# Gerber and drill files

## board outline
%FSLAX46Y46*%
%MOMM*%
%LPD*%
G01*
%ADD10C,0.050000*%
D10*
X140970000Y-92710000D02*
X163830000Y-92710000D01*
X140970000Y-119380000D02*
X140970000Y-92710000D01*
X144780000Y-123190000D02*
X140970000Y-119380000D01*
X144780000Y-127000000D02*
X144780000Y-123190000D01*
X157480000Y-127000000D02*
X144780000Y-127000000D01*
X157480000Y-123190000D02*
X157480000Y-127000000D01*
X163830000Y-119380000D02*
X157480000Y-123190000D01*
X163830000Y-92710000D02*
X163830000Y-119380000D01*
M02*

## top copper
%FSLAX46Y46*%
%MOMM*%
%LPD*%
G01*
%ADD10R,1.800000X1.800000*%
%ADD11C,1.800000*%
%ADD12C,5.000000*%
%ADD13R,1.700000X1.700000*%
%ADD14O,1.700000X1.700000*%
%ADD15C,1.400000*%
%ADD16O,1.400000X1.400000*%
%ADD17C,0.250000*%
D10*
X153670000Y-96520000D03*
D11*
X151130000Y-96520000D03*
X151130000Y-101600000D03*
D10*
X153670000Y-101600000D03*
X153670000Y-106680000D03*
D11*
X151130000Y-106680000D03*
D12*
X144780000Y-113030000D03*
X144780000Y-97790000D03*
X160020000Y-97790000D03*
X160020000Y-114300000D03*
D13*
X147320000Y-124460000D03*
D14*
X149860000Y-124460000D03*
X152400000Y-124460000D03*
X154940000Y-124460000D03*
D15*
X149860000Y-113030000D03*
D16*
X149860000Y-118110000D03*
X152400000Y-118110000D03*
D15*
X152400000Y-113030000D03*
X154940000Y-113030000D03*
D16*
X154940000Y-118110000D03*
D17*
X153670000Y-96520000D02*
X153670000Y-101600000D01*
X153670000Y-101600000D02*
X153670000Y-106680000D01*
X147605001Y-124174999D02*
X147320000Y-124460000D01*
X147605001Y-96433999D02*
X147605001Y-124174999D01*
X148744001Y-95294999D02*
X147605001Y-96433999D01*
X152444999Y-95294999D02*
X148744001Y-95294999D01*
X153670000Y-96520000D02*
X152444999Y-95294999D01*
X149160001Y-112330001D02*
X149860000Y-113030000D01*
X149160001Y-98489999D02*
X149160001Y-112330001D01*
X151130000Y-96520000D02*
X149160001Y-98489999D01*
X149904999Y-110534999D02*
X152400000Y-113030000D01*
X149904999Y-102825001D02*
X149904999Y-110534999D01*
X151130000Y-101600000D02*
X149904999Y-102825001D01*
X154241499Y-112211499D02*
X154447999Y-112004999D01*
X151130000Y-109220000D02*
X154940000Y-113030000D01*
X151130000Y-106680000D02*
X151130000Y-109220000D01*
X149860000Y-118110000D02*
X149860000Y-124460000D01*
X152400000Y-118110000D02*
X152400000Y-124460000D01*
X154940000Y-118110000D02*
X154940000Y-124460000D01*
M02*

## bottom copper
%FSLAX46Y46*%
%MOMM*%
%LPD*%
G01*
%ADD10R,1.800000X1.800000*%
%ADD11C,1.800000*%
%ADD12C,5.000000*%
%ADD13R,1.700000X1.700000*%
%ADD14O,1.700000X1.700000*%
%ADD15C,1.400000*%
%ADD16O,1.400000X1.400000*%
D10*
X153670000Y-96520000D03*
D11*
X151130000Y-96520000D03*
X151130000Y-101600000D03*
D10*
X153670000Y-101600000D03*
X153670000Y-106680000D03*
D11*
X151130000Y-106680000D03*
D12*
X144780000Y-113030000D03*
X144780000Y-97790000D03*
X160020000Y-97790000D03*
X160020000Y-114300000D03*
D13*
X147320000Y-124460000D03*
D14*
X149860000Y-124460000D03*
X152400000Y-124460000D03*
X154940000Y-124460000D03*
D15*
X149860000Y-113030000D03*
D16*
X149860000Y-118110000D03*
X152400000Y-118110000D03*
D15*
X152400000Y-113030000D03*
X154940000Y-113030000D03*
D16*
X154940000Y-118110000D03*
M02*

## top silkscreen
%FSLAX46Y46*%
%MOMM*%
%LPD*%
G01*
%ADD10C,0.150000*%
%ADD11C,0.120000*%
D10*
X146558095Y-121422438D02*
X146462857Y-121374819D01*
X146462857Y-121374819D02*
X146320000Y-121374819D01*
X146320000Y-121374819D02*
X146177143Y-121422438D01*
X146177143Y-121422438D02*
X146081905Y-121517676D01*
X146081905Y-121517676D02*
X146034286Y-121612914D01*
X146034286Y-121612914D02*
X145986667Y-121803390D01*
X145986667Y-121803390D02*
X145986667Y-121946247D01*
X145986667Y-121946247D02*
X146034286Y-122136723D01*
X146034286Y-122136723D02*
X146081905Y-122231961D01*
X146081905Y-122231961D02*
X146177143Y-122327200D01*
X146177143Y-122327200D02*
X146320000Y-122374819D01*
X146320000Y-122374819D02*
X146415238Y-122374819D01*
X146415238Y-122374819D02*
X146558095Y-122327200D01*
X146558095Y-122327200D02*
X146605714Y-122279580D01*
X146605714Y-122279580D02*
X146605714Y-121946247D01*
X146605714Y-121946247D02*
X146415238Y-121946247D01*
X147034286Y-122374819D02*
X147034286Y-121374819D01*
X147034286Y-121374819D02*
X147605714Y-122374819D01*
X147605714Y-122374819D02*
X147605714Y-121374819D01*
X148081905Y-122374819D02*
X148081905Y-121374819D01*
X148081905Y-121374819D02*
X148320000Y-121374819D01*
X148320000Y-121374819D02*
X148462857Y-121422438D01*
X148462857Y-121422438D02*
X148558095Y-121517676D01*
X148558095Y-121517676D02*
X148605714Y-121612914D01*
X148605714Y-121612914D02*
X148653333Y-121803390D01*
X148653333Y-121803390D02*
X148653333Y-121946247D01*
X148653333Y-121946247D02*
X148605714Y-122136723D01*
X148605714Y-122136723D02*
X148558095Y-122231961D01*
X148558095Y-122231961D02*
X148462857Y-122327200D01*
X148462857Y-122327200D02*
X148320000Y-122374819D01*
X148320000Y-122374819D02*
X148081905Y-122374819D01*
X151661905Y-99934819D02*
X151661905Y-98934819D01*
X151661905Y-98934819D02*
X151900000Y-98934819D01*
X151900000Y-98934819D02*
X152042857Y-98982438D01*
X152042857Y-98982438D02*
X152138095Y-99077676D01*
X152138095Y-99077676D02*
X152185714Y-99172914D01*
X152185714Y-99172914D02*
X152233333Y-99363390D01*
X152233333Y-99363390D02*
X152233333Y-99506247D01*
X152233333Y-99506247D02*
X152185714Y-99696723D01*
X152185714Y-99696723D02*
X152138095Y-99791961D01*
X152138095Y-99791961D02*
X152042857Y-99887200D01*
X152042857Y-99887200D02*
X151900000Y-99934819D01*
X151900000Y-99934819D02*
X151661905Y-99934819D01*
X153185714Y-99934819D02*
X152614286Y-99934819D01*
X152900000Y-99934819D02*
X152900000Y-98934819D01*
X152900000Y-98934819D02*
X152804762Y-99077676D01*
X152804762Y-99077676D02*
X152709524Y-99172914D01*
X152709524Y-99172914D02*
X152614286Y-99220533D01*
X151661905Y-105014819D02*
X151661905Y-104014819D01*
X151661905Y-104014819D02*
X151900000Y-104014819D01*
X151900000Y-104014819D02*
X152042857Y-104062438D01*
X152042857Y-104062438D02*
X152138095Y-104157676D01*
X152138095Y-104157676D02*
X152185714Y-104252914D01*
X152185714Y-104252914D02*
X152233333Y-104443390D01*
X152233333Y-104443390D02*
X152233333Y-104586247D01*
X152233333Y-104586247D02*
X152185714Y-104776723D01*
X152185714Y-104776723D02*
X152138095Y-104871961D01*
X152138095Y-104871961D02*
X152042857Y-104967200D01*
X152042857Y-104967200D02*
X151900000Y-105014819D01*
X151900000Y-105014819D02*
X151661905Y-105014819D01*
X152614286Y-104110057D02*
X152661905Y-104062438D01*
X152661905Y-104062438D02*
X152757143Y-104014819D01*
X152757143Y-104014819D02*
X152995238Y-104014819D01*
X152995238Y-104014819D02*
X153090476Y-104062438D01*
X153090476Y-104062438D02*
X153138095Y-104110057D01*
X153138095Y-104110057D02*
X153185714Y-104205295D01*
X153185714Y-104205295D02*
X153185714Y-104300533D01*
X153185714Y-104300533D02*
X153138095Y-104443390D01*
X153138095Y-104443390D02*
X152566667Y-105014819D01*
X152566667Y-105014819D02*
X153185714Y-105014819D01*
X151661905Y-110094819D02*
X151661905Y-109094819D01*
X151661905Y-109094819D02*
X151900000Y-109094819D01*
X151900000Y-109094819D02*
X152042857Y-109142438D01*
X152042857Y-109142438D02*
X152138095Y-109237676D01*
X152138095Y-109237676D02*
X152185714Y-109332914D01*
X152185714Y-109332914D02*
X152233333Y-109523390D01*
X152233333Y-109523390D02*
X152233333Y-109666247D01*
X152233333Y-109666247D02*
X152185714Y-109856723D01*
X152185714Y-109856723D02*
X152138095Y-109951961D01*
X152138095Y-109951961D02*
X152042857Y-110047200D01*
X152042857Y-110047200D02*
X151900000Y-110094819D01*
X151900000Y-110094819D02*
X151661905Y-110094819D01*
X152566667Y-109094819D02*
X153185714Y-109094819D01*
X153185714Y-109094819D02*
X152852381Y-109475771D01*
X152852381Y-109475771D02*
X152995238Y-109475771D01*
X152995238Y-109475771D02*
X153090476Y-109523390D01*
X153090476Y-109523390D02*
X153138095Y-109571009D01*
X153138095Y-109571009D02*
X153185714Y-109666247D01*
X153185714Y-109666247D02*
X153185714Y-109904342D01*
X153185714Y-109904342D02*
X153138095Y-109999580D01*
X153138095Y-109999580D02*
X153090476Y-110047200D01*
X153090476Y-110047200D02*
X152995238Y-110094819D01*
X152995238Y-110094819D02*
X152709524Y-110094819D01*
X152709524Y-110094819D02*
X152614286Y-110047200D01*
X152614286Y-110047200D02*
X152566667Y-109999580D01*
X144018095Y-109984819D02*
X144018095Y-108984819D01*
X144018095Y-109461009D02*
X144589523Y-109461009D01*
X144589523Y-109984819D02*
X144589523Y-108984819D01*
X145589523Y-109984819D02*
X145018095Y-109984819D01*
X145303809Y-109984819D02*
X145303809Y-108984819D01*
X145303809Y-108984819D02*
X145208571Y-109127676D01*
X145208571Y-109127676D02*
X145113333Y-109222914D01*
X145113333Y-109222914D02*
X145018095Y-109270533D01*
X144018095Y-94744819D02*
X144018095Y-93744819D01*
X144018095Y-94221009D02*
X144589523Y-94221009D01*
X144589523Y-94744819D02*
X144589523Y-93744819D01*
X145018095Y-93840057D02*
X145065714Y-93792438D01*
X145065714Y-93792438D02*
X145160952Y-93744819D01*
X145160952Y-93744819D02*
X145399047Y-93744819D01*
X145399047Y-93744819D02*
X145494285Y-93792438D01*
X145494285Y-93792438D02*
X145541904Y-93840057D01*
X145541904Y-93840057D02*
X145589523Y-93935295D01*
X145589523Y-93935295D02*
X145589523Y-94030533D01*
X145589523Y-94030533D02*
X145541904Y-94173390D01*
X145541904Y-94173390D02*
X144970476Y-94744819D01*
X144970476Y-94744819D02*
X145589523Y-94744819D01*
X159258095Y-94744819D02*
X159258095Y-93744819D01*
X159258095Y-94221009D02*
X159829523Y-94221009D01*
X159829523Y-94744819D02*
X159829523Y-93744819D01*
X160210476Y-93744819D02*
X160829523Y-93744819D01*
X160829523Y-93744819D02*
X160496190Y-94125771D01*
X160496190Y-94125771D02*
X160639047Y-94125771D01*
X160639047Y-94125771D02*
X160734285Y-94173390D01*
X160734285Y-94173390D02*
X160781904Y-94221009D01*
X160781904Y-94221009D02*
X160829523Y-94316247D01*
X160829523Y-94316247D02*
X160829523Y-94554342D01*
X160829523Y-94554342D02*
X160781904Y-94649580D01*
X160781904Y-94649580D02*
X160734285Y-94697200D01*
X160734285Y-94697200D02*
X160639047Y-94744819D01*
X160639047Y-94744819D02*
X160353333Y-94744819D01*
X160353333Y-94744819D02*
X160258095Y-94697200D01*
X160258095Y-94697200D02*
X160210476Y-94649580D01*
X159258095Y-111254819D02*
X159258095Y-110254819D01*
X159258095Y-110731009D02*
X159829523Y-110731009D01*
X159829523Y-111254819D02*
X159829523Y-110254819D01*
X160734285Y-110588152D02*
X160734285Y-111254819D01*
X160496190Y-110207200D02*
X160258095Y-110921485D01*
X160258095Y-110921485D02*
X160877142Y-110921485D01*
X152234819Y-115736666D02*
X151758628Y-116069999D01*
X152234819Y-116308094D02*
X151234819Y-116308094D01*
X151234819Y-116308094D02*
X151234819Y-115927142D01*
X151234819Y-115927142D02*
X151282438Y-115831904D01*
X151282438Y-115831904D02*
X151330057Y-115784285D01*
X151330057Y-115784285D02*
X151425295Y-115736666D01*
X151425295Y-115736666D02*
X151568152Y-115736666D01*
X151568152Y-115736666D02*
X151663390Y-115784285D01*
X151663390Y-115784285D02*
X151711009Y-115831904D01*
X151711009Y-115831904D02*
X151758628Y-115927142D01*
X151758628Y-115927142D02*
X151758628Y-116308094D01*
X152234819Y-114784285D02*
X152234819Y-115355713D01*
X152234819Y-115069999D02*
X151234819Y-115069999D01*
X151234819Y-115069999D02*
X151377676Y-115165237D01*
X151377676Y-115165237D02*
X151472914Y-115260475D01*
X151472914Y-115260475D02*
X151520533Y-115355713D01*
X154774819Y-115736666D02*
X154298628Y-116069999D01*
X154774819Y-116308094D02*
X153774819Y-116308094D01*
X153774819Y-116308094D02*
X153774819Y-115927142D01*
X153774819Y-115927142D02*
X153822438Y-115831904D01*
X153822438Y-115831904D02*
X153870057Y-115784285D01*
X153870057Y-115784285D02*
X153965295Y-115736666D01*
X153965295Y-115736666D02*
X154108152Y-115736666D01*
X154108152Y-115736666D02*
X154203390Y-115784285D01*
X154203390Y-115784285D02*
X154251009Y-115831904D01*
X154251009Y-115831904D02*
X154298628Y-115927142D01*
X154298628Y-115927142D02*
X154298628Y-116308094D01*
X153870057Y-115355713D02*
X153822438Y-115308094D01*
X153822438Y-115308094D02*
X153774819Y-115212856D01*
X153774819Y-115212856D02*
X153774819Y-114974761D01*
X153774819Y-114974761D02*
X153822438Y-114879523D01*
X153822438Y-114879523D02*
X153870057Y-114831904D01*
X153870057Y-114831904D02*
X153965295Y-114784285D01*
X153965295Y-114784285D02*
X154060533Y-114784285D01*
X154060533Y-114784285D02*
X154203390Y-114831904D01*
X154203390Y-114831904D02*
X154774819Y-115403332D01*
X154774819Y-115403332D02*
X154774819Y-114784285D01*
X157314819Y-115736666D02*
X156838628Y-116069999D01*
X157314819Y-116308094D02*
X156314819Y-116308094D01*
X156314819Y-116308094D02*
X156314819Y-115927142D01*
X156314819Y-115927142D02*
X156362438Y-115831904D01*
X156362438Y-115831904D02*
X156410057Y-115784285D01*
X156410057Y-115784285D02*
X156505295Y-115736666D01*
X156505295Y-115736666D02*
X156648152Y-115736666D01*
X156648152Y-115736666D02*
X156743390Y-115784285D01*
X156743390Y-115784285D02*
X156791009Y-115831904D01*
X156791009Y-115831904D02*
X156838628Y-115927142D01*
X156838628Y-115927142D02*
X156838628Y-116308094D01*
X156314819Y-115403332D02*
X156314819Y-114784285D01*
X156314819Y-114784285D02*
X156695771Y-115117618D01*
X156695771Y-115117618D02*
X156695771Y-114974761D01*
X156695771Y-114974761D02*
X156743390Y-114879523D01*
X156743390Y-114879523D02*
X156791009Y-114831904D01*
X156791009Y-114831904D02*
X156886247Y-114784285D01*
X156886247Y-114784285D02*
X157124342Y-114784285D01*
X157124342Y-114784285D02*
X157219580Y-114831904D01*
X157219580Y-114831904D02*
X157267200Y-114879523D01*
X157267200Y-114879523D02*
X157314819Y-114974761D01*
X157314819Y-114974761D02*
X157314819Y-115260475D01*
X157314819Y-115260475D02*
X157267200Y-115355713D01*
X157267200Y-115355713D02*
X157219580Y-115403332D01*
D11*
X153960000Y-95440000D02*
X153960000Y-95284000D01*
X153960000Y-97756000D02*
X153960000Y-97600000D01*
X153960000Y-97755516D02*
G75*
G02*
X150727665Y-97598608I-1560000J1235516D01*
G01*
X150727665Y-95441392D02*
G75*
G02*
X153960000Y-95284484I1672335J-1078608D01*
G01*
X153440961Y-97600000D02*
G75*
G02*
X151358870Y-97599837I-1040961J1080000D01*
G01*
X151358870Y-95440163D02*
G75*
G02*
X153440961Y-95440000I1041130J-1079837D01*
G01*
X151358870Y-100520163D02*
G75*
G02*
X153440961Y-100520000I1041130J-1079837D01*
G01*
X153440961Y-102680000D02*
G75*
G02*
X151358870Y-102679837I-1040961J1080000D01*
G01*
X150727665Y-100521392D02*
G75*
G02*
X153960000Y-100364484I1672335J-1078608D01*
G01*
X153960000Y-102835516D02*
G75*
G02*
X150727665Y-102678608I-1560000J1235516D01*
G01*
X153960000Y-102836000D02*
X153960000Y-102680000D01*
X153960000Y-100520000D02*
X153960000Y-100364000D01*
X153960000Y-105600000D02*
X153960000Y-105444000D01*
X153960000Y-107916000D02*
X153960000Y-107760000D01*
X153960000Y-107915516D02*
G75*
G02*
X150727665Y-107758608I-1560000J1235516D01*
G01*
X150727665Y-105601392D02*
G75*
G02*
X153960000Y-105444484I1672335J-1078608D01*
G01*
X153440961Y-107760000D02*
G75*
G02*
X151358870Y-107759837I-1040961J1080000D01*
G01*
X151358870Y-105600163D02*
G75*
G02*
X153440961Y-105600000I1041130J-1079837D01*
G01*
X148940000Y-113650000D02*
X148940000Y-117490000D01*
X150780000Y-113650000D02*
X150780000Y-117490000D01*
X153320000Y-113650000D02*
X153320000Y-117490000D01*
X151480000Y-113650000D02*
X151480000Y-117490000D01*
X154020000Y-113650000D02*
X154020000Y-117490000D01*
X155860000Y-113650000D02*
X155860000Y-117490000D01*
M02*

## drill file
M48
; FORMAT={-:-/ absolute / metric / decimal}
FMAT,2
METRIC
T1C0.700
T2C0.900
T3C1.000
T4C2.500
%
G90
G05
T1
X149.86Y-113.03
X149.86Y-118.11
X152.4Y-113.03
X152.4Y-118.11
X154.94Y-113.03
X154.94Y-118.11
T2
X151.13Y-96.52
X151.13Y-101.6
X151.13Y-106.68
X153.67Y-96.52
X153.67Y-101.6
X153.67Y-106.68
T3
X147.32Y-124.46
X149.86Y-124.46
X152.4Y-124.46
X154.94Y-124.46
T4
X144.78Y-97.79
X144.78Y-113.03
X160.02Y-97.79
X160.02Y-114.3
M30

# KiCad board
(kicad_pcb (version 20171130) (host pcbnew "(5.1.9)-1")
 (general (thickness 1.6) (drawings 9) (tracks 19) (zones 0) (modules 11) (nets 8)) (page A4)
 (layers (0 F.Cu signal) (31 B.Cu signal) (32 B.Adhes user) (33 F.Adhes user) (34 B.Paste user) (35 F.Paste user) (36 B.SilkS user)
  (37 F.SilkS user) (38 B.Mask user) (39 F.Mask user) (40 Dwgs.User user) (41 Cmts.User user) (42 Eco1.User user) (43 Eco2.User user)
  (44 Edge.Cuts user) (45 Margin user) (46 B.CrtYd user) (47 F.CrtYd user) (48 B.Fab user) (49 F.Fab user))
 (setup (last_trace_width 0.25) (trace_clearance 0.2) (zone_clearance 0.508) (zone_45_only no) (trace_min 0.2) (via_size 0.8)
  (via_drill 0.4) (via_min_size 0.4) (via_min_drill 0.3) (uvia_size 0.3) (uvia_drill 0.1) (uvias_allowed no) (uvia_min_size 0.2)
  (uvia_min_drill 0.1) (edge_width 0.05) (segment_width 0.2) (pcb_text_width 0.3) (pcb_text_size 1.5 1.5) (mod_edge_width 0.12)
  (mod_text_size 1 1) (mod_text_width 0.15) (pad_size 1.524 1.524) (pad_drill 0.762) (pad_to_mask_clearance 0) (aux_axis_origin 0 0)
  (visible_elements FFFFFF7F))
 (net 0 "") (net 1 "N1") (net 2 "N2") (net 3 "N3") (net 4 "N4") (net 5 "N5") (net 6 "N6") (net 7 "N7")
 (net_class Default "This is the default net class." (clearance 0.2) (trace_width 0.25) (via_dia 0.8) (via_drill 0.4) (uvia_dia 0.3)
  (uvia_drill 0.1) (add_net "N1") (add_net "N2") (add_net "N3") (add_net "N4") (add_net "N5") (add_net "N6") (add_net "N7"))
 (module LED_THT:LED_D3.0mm (layer F.Cu) (at 153.67 96.52 180)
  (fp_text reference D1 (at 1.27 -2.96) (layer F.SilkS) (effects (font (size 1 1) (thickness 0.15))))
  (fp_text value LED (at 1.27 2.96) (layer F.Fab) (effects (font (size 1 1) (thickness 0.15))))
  (fp_line (start -0.29 1.08) (end -0.29 1.236) (layer F.SilkS) (width 0.12))
  (fp_line (start -0.29 -1.236) (end -0.29 -1.08) (layer F.SilkS) (width 0.12))
  (fp_arc (start 1.27 0) (end -0.29 -1.235516) (angle 108.8) (layer F.SilkS) (width 0.12))
  (fp_arc (start 1.27 0) (end -0.29 1.235516) (angle -108.8) (layer F.SilkS) (width 0.12))
  (fp_arc (start 1.27 0) (end 0.229039 -1.08) (angle 87.9) (layer F.SilkS) (width 0.12))
  (fp_arc (start 1.27 0) (end 0.229039 1.08) (angle -87.9) (layer F.SilkS) (width 0.12))
  (pad 1 thru_hole rect (at 0 0 180) (size 1.8 1.8) (drill 0.9) (layers *.Cu *.Mask) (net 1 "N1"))
  (pad 2 thru_hole circle (at 2.54 0 180) (size 1.8 1.8) (drill 0.9) (layers *.Cu *.Mask) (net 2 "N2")))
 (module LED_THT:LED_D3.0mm (layer F.Cu) (at 153.67 101.6 180)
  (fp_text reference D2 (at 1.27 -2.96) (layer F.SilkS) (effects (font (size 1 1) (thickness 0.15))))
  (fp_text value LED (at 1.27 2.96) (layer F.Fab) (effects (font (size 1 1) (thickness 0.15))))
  (fp_arc (start 1.27 0) (end 0.229039 1.08) (angle -87.9) (layer F.SilkS) (width 0.12))
  (fp_arc (start 1.27 0) (end 0.229039 -1.08) (angle 87.9) (layer F.SilkS) (width 0.12))
  (fp_arc (start 1.27 0) (end -0.29 1.235516) (angle -108.8) (layer F.SilkS) (width 0.12))
  (fp_arc (start 1.27 0) (end -0.29 -1.235516) (angle 108.8) (layer F.SilkS) (width 0.12))
  (fp_line (start -0.29 -1.236) (end -0.29 -1.08) (layer F.SilkS) (width 0.12))
  (fp_line (start -0.29 1.08) (end -0.29 1.236) (layer F.SilkS) (width 0.12))
  (pad 2 thru_hole circle (at 2.54 0 180) (size 1.8 1.8) (drill 0.9) (layers *.Cu *.Mask) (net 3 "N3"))
  (pad 1 thru_hole rect (at 0 0 180) (size 1.8 1.8) (drill 0.9) (layers *.Cu *.Mask) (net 1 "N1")))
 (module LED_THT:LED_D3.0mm (layer F.Cu) (at 153.67 106.68 180)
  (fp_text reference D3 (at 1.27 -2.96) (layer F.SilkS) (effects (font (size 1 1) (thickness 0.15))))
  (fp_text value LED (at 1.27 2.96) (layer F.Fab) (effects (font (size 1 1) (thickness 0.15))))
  (fp_line (start -0.29 1.08) (end -0.29 1.236) (layer F.SilkS) (width 0.12))
  (fp_line (start -0.29 -1.236) (end -0.29 -1.08) (layer F.SilkS) (width 0.12))
  (fp_arc (start 1.27 0) (end -0.29 -1.235516) (angle 108.8) (layer F.SilkS) (width 0.12))
  (fp_arc (start 1.27 0) (end -0.29 1.235516) (angle -108.8) (layer F.SilkS) (width 0.12))
  (fp_arc (start 1.27 0) (end 0.229039 -1.08) (angle 87.9) (layer F.SilkS) (width 0.12))
  (fp_arc (start 1.27 0) (end 0.229039 1.08) (angle -87.9) (layer F.SilkS) (width 0.12))
  (pad 1 thru_hole rect (at 0 0 180) (size 1.8 1.8) (drill 0.9) (layers *.Cu *.Mask) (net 1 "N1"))
  (pad 2 thru_hole circle (at 2.54 0 180) (size 1.8 1.8) (drill 0.9) (layers *.Cu *.Mask) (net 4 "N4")))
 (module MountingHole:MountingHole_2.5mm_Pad (layer F.Cu) (at 144.78 113.03)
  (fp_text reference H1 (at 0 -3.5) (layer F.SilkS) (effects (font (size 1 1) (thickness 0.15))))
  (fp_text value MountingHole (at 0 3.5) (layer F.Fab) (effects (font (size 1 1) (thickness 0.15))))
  (pad 1 thru_hole circle (at 0 0) (size 5 5) (drill 2.5) (layers *.Cu *.Mask)))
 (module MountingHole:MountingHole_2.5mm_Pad (layer F.Cu) (at 144.78 97.79)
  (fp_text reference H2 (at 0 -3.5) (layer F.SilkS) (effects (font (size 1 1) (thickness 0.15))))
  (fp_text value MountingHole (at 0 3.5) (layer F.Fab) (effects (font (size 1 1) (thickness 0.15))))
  (pad 1 thru_hole circle (at 0 0) (size 5 5) (drill 2.5) (layers *.Cu *.Mask)))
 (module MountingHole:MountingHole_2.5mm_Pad (layer F.Cu) (at 160.02 97.79)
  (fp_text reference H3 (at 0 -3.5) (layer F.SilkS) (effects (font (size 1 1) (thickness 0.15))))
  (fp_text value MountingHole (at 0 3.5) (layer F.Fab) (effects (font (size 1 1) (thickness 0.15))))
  (pad 1 thru_hole circle (at 0 0) (size 5 5) (drill 2.5) (layers *.Cu *.Mask)))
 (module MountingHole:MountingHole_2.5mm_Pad (layer F.Cu) (at 160.02 114.3)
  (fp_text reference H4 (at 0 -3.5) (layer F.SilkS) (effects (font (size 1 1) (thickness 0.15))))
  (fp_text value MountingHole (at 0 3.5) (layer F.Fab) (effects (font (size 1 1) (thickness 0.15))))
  (pad 1 thru_hole circle (at 0 0) (size 5 5) (drill 2.5) (layers *.Cu *.Mask)))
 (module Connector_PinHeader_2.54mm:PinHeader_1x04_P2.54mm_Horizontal (layer B.Cu) (at 147.32 124.46 270)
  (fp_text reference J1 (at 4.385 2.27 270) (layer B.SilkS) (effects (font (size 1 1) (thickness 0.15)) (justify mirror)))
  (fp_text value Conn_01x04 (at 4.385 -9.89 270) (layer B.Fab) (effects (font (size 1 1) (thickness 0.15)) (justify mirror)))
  (pad 1 thru_hole rect (at 0 0 270) (size 1.7 1.7) (drill 1) (layers *.Cu *.Mask) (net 1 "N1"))
  (pad 2 thru_hole oval (at 0 -2.54 270) (size 1.7 1.7) (drill 1) (layers *.Cu *.Mask) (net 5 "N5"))
  (pad 3 thru_hole oval (at 0 -5.08 270) (size 1.7 1.7) (drill 1) (layers *.Cu *.Mask) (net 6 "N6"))
  (pad 4 thru_hole oval (at 0 -7.62 270) (size 1.7 1.7) (drill 1) (layers *.Cu *.Mask) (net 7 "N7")))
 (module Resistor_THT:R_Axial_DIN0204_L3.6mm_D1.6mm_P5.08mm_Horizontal (layer F.Cu) (at 149.86 113.03 270)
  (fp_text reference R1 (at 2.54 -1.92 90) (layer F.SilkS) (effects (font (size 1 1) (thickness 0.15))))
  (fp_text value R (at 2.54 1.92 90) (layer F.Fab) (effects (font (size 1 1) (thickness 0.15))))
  (fp_line (start 0.62 0.92) (end 4.46 0.92) (layer F.SilkS) (width 0.12))
  (fp_line (start 0.62 -0.92) (end 4.46 -0.92) (layer F.SilkS) (width 0.12))
  (pad 1 thru_hole circle (at 0 0 270) (size 1.4 1.4) (drill 0.7) (layers *.Cu *.Mask) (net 2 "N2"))
  (pad 2 thru_hole oval (at 5.08 0 270) (size 1.4 1.4) (drill 0.7) (layers *.Cu *.Mask) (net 5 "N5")))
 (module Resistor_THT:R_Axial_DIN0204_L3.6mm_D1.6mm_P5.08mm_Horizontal (layer F.Cu) (at 152.4 113.03 270)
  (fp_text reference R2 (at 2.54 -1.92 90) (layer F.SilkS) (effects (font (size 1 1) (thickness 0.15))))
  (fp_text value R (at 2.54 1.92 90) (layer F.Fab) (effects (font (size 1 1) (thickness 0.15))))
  (fp_line (start 0.62 -0.92) (end 4.46 -0.92) (layer F.SilkS) (width 0.12))
  (fp_line (start 0.62 0.92) (end 4.46 0.92) (layer F.SilkS) (width 0.12))
  (pad 2 thru_hole oval (at 5.08 0 270) (size 1.4 1.4) (drill 0.7) (layers *.Cu *.Mask) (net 6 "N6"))
  (pad 1 thru_hole circle (at 0 0 270) (size 1.4 1.4) (drill 0.7) (layers *.Cu *.Mask) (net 3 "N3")))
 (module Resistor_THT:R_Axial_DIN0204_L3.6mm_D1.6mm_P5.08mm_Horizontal (layer F.Cu) (at 154.94 113.03 270)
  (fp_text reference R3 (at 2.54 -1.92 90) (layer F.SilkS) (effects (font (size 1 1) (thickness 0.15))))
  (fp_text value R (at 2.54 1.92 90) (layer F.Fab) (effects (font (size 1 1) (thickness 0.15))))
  (fp_line (start 0.62 0.92) (end 4.46 0.92) (layer F.SilkS) (width 0.12))
  (fp_line (start 0.62 -0.92) (end 4.46 -0.92) (layer F.SilkS) (width 0.12))
  (pad 1 thru_hole circle (at 0 0 270) (size 1.4 1.4) (drill 0.7) (layers *.Cu *.Mask) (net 4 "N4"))
  (pad 2 thru_hole oval (at 5.08 0 270) (size 1.4 1.4) (drill 0.7) (layers *.Cu *.Mask) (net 7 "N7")))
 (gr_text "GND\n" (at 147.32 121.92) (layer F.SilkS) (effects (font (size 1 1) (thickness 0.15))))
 (gr_line (start 140.97 92.71) (end 163.83 92.71) (layer Edge.Cuts) (width 0.05))
 (gr_line (start 140.97 119.38) (end 140.97 92.71) (layer Edge.Cuts) (width 0.05))
 (gr_line (start 144.78 123.19) (end 140.97 119.38) (layer Edge.Cuts) (width 0.05))
 (gr_line (start 144.78 127) (end 144.78 123.19) (layer Edge.Cuts) (width 0.05))
 (gr_line (start 157.48 127) (end 144.78 127) (layer Edge.Cuts) (width 0.05))
 (gr_line (start 157.48 123.19) (end 157.48 127) (layer Edge.Cuts) (width 0.05))
 (gr_line (start 163.83 119.38) (end 157.48 123.19) (layer Edge.Cuts) (width 0.05))
 (gr_line (start 163.83 92.71) (end 163.83 119.38) (layer Edge.Cuts) (width 0.05))
 (segment (start 153.67 96.52) (end 153.67 101.6) (width 0.25) (layer F.Cu) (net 1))
 (segment (start 153.67 101.6) (end 153.67 106.68) (width 0.25) (layer F.Cu) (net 1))
 (segment (start 147.605001 124.174999) (end 147.32 124.46) (width 0.25) (layer F.Cu) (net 1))
 (segment (start 147.605001 96.433999) (end 147.605001 124.174999) (width 0.25) (layer F.Cu) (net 1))
 (segment (start 148.744001 95.294999) (end 147.605001 96.433999) (width 0.25) (layer F.Cu) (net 1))
 (segment (start 152.444999 95.294999) (end 148.744001 95.294999) (width 0.25) (layer F.Cu) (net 1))
 (segment (start 153.67 96.52) (end 152.444999 95.294999) (width 0.25) (layer F.Cu) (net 1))
 (segment (start 149.160001 112.330001) (end 149.86 113.03) (width 0.25) (layer F.Cu) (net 2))
 (segment (start 149.160001 98.489999) (end 149.160001 112.330001) (width 0.25) (layer F.Cu) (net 2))
 (segment (start 151.13 96.52) (end 149.160001 98.489999) (width 0.25) (layer F.Cu) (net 2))
 (segment (start 149.904999 110.534999) (end 152.4 113.03) (width 0.25) (layer F.Cu) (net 3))
 (segment (start 149.904999 102.825001) (end 149.904999 110.534999) (width 0.25) (layer F.Cu) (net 3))
 (segment (start 151.13 101.6) (end 149.904999 102.825001) (width 0.25) (layer F.Cu) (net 3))
 (segment (start 154.241499 112.211499) (end 154.447999 112.004999) (width 0.25) (layer F.Cu) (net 4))
 (segment (start 151.13 109.22) (end 154.94 113.03) (width 0.25) (layer F.Cu) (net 4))
 (segment (start 151.13 106.68) (end 151.13 109.22) (width 0.25) (layer F.Cu) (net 4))
 (segment (start 149.86 118.11) (end 149.86 124.46) (width 0.25) (layer F.Cu) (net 5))
 (segment (start 152.4 118.11) (end 152.4 124.46) (width 0.25) (layer F.Cu) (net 6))
 (segment (start 154.94 118.11) (end 154.94 124.46) (width 0.25) (layer F.Cu) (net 7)))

